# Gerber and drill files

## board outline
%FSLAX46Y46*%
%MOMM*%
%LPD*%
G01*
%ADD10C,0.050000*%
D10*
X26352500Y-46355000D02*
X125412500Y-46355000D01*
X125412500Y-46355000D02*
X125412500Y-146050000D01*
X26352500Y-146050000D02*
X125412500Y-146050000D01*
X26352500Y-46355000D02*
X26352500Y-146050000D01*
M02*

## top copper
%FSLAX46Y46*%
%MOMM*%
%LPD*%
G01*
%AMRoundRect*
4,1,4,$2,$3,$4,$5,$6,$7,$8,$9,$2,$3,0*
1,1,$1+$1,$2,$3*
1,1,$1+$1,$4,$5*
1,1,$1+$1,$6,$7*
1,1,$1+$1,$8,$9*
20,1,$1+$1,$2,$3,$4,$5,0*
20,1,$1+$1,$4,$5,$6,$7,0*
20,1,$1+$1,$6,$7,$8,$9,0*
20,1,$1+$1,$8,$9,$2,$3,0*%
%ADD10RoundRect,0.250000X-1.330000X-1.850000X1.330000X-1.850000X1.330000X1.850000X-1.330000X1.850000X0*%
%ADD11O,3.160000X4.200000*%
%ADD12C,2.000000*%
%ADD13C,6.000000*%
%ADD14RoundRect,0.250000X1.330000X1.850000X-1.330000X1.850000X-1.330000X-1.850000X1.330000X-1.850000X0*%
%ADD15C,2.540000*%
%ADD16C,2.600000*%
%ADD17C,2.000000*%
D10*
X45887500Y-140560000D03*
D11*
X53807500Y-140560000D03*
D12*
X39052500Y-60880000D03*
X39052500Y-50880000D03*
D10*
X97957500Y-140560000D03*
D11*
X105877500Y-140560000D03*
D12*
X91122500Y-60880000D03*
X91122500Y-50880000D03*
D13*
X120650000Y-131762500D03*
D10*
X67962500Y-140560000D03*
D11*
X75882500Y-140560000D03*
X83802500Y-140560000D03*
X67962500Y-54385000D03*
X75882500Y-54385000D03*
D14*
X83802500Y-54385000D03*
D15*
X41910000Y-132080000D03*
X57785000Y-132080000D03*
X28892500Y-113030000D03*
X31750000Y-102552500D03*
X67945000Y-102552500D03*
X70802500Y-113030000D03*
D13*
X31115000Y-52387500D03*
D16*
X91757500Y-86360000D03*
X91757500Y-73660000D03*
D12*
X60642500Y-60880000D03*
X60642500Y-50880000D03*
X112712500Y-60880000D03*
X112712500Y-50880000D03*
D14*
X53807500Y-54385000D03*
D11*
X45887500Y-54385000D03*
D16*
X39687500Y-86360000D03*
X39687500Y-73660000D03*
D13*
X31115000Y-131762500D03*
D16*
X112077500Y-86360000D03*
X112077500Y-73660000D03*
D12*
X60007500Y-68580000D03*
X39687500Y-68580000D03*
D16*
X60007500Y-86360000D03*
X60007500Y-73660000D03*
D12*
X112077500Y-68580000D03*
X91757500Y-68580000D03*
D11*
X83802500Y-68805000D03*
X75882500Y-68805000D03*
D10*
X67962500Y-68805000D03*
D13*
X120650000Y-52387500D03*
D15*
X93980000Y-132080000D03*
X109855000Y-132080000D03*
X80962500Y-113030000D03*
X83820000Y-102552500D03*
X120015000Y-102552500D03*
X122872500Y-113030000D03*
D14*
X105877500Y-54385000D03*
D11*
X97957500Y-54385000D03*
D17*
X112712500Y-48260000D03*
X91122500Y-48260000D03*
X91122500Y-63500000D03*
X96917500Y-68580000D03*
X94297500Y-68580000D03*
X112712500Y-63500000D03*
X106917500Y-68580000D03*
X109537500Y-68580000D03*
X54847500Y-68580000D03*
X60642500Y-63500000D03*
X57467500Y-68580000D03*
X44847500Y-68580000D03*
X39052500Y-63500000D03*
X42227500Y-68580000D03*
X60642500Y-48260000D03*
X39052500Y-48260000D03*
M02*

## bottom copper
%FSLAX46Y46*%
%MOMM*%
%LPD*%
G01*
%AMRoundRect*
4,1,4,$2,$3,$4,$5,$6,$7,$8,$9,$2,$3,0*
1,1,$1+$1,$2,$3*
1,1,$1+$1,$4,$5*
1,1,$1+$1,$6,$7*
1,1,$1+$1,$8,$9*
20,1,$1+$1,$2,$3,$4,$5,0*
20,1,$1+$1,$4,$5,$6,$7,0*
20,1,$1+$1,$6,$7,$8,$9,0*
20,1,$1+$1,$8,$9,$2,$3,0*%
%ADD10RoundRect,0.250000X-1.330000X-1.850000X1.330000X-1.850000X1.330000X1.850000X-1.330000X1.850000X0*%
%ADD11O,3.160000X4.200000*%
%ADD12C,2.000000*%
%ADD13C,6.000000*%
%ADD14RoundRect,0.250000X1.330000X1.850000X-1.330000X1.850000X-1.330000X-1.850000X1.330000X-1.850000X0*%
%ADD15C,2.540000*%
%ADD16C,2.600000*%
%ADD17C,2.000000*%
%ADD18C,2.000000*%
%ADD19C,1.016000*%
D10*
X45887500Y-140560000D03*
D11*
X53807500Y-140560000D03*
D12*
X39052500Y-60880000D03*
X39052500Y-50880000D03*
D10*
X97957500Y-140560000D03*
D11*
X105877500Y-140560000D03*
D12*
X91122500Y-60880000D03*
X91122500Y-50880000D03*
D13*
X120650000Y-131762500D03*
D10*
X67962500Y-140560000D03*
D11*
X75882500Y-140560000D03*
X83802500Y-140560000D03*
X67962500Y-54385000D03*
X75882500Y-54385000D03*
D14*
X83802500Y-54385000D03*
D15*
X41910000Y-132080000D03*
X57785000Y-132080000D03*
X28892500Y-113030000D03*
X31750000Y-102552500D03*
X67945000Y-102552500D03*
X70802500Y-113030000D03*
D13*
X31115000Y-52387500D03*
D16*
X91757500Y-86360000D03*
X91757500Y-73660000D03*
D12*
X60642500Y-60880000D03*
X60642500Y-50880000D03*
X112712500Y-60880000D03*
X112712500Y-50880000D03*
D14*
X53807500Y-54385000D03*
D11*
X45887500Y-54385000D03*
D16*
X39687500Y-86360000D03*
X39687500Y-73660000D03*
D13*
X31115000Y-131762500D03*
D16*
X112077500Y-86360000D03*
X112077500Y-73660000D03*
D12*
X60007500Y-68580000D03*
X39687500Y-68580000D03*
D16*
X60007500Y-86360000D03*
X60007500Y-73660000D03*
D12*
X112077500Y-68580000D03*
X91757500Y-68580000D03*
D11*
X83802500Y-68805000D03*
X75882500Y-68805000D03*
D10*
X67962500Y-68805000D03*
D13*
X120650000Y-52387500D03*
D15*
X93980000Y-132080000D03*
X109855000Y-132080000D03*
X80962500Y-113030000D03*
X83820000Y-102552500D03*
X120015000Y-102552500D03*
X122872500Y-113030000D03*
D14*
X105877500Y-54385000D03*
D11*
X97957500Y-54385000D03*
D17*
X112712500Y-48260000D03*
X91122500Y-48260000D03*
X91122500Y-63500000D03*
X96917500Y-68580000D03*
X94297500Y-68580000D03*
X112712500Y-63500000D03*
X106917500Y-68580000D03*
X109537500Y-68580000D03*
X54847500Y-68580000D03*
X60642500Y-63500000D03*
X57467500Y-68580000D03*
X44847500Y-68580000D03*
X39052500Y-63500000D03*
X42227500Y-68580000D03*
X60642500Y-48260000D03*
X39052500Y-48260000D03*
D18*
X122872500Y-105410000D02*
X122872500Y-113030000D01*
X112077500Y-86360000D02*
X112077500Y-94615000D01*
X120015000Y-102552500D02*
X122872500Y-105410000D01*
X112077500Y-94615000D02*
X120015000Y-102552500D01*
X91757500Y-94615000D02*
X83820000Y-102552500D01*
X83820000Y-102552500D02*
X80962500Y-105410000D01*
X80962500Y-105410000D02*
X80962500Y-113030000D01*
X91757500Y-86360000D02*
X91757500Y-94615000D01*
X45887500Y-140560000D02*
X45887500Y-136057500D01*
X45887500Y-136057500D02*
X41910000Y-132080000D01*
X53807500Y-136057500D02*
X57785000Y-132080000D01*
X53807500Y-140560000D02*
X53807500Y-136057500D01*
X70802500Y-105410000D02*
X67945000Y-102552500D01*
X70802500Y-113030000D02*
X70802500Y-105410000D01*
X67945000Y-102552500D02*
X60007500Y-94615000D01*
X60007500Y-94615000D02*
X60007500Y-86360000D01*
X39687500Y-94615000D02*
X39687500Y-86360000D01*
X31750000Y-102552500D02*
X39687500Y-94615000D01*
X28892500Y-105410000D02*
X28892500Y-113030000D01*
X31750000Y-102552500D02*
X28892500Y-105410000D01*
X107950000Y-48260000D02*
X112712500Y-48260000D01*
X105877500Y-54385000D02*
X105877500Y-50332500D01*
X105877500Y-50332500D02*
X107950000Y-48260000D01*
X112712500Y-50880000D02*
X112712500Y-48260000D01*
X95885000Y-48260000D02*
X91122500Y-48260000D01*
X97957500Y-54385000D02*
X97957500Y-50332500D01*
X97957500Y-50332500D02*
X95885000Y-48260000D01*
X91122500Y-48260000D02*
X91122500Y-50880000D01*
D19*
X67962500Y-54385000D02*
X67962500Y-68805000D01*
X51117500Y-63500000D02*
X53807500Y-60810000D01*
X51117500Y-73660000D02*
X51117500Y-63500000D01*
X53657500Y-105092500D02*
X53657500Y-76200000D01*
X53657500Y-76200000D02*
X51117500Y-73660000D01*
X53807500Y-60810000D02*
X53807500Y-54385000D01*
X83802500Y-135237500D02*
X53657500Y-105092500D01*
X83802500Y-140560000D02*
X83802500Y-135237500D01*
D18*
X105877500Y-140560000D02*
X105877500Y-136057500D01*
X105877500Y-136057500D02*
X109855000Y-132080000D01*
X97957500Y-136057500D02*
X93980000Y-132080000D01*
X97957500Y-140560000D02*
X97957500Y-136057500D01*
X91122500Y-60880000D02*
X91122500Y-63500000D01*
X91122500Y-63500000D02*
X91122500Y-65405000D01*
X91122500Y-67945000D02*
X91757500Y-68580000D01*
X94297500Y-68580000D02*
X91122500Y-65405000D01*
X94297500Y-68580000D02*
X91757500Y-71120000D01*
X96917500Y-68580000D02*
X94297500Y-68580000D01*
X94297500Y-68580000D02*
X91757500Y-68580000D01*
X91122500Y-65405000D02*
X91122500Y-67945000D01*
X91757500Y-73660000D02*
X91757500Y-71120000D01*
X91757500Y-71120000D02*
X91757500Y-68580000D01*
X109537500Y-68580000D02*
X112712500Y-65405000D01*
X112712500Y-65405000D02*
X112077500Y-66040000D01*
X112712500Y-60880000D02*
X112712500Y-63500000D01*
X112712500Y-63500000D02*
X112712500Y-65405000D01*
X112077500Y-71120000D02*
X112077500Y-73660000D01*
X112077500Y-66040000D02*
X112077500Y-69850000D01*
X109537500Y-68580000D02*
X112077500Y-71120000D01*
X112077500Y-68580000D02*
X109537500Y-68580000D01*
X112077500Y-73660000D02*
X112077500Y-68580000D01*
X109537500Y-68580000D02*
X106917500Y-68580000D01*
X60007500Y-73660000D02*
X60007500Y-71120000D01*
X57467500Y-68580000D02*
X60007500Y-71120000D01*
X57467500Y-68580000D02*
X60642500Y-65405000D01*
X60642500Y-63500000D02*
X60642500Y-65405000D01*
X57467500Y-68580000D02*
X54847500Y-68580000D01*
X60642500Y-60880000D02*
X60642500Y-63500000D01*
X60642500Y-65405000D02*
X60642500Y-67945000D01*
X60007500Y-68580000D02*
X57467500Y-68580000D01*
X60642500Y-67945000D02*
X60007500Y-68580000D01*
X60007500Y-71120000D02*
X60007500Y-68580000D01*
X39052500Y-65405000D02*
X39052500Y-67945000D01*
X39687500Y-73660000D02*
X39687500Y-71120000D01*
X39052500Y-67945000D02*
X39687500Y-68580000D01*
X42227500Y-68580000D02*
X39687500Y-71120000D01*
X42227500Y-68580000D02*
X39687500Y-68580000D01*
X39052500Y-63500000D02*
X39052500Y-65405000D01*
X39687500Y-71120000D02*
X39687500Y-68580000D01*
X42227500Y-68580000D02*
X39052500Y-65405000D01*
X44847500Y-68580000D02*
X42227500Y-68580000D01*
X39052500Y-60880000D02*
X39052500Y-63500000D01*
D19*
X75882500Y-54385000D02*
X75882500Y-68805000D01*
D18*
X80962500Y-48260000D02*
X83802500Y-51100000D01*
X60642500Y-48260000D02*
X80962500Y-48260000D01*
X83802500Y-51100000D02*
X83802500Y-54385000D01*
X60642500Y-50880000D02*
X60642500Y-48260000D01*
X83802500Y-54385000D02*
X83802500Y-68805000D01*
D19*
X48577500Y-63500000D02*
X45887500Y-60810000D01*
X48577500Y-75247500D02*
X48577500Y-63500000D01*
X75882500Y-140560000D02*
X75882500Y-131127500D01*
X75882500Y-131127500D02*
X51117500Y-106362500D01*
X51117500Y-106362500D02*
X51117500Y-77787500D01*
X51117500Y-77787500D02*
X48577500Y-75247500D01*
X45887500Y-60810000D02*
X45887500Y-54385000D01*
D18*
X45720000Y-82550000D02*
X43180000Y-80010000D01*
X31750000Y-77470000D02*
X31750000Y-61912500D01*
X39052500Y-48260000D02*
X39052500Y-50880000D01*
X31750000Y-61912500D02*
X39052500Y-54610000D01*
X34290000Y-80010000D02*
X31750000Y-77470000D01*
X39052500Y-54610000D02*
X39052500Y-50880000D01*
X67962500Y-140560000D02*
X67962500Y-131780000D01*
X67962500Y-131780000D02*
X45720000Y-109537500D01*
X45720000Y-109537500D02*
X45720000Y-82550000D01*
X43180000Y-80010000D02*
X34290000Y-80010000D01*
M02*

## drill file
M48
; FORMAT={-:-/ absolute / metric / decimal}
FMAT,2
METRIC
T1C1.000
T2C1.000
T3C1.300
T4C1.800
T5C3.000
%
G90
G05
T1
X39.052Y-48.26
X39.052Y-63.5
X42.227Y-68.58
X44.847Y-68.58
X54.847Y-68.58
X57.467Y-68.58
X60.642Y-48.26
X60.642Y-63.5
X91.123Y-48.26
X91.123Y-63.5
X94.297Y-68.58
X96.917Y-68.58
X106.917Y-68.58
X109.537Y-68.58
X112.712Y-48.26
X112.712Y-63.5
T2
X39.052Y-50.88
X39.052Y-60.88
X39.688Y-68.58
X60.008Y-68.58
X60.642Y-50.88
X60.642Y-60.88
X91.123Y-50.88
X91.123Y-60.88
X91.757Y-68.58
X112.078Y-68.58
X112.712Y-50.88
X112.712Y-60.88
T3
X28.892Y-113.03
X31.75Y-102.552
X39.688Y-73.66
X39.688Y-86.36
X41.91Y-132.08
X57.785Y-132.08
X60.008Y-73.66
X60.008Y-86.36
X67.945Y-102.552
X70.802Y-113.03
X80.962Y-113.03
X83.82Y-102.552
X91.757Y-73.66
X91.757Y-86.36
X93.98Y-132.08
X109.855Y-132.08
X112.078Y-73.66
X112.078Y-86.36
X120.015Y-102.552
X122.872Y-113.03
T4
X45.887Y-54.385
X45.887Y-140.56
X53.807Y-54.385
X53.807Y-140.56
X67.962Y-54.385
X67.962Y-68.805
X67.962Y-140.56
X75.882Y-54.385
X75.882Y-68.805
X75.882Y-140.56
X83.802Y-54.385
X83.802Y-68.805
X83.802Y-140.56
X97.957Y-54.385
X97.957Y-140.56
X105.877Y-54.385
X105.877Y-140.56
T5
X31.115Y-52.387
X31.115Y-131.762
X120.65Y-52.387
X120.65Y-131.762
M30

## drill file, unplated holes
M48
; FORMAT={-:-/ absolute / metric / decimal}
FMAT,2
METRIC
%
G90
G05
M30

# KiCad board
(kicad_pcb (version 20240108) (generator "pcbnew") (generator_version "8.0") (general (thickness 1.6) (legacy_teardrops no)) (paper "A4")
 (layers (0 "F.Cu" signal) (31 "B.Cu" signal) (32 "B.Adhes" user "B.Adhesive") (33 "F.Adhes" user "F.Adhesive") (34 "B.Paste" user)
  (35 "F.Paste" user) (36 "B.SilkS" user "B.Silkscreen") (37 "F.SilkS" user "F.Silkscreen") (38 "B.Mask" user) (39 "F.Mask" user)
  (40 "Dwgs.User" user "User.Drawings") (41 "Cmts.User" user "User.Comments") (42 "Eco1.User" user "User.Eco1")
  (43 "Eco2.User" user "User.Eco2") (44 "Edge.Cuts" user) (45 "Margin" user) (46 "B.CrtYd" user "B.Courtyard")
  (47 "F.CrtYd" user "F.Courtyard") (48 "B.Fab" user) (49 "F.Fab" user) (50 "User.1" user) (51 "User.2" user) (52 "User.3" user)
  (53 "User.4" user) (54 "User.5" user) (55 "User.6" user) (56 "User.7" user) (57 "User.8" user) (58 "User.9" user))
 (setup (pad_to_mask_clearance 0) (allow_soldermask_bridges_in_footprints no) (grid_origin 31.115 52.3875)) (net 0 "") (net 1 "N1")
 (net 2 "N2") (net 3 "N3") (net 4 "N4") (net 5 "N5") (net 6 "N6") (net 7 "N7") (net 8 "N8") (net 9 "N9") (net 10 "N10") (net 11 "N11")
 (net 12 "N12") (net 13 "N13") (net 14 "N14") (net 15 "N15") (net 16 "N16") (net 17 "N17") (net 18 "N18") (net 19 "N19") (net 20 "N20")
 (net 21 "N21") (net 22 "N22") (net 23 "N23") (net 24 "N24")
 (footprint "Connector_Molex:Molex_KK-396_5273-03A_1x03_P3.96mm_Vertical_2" (layer "F.Cu") (at 45.8875 140.56)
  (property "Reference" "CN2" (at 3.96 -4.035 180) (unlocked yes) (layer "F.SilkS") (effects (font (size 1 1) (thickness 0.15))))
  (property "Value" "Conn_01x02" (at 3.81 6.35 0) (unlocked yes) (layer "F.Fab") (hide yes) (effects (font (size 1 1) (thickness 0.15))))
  (pad "1" thru_hole roundrect (at 0 0) (size 3.16 4.2) (drill 1.8) (layers "*.Cu" "*.Mask") (remove_unused_layers no)
   (roundrect_rratio 0.079114) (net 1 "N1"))
  (pad "2" thru_hole oval (at 7.92 0) (size 3.16 4.2) (drill 1.8) (layers "*.Cu" "*.Mask") (remove_unused_layers no) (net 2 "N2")))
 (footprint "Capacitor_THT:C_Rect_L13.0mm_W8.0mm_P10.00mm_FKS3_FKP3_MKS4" (layer "F.Cu") (at 39.0525 60.88 90)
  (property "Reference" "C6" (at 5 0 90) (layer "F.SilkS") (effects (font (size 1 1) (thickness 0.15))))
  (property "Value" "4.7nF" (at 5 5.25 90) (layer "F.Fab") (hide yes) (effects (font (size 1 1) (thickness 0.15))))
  (pad "1" thru_hole circle (at 0 0 90) (size 2 2) (drill 1) (layers "*.Cu" "*.Mask") (remove_unused_layers no) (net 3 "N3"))
  (pad "2" thru_hole circle (at 10 0 90) (size 2 2) (drill 1) (layers "*.Cu" "*.Mask") (remove_unused_layers no) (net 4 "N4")))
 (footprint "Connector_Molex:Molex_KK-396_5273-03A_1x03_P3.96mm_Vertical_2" (layer "F.Cu") (at 97.9575 140.56)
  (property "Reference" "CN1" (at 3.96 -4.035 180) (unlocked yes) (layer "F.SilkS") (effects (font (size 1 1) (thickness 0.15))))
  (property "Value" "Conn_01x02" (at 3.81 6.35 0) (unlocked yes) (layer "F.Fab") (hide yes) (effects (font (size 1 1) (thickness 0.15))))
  (pad "1" thru_hole roundrect (at 0 0) (size 3.16 4.2) (drill 1.8) (layers "*.Cu" "*.Mask") (remove_unused_layers no)
   (roundrect_rratio 0.079114) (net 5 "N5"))
  (pad "2" thru_hole oval (at 7.92 0) (size 3.16 4.2) (drill 1.8) (layers "*.Cu" "*.Mask") (remove_unused_layers no) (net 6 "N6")))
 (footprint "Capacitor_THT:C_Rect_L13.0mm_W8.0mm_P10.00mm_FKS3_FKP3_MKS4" (layer "F.Cu") (at 91.1225 60.88 90)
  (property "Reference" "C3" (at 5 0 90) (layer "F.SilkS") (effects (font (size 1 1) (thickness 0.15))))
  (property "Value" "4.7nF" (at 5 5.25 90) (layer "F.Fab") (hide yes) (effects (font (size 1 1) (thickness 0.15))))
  (pad "1" thru_hole circle (at 0 0 90) (size 2 2) (drill 1) (layers "*.Cu" "*.Mask") (remove_unused_layers no) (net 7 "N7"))
  (pad "2" thru_hole circle (at 10 0 90) (size 2 2) (drill 1) (layers "*.Cu" "*.Mask") (remove_unused_layers no) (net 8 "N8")))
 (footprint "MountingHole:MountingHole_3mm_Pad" (layer "F.Cu") (at 120.65 131.7625 -90)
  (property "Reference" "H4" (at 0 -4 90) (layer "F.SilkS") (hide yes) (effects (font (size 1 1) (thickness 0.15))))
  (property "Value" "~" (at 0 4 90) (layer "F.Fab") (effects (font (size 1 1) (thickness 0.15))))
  (pad "1" thru_hole circle (at 0 0 270) (size 6 6) (drill 3) (layers "*.Cu" "*.Mask") (remove_unused_layers no) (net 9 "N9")))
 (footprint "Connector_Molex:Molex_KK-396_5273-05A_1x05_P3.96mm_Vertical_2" (layer "F.Cu") (at 67.9625 140.56)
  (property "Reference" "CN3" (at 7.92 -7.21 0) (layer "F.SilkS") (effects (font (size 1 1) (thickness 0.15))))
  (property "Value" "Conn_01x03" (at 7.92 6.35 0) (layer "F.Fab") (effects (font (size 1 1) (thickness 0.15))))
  (pad "1" thru_hole roundrect (at 0 0) (size 3.16 4.2) (drill 1.8) (layers "*.Cu" "*.Mask") (remove_unused_layers no)
   (roundrect_rratio 0.079114) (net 4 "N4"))
  (pad "2" thru_hole oval (at 7.92 0) (size 3.16 4.2) (drill 1.8) (layers "*.Cu" "*.Mask") (remove_unused_layers no) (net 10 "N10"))
  (pad "3" thru_hole oval (at 15.84 0) (size 3.16 4.2) (drill 1.8) (layers "*.Cu" "*.Mask") (remove_unused_layers no) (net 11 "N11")))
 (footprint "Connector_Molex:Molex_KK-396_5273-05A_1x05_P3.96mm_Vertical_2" (layer "F.Cu") (at 83.8025 54.385 180)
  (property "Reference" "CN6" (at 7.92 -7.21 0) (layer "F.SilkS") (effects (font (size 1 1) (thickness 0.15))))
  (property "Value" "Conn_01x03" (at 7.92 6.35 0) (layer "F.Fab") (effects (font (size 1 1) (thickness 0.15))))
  (pad "1" thru_hole roundrect (at 0 0 180) (size 3.16 4.2) (drill 1.8) (layers "*.Cu" "*.Mask") (remove_unused_layers no)
   (roundrect_rratio 0.079114) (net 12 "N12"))
  (pad "2" thru_hole oval (at 7.92 0 180) (size 3.16 4.2) (drill 1.8) (layers "*.Cu" "*.Mask") (remove_unused_layers no) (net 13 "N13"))
  (pad "3" thru_hole oval (at 15.84 0 180) (size 3.16 4.2) (drill 1.8) (layers "*.Cu" "*.Mask") (remove_unused_layers no) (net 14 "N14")))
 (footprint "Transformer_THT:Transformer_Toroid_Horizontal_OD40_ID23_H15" (layer "F.Cu") (at 49.8475 113.03)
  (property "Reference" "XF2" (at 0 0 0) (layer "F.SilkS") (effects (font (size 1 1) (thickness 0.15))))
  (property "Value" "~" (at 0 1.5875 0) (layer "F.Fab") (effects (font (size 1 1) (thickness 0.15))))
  (pad "1" thru_hole circle (at -7.9375 19.05) (size 2.54 2.54) (drill 1.3) (layers "*.Cu" "*.Mask") (remove_unused_layers no) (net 1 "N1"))
  (pad "2" thru_hole circle (at 7.9375 19.05) (size 2.54 2.54) (drill 1.3) (layers "*.Cu" "*.Mask") (remove_unused_layers no) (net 2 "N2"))
  (pad "3" thru_hole circle (at -20.955 0) (size 2.54 2.54) (drill 1.3) (layers "*.Cu" "*.Mask") (remove_unused_layers no) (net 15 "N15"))
  (pad "3" thru_hole circle (at -18.0975 -10.4775) (size 2.54 2.54) (drill 1.3) (layers "*.Cu" "*.Mask") (remove_unused_layers no)
   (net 15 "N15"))
  (pad "4" thru_hole circle (at 18.0975 -10.4775) (size 2.54 2.54) (drill 1.3) (layers "*.Cu" "*.Mask") (remove_unused_layers no)
   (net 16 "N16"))
  (pad "4" thru_hole circle (at 20.955 0) (size 2.54 2.54) (drill 1.3) (layers "*.Cu" "*.Mask") (remove_unused_layers no) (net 16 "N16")))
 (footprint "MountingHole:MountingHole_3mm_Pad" (layer "F.Cu") (at 31.115 52.3875 -90)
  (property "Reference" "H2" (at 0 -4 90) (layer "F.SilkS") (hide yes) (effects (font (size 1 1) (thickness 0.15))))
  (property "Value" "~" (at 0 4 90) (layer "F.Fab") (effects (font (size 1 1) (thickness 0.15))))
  (pad "1" thru_hole circle (at 0 0 270) (size 6 6) (drill 3) (layers "*.Cu" "*.Mask") (remove_unused_layers no) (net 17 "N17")))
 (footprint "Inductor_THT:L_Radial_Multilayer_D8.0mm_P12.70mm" (layer "F.Cu") (at 91.7575 81.915 90)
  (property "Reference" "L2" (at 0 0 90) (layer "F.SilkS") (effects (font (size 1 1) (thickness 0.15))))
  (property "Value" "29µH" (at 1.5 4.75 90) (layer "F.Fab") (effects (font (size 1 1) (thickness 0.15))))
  (pad "1" thru_hole circle (at -4.445 0 90) (size 2.6 2.6) (drill 1.3) (layers "*.Cu" "*.Mask") (remove_unused_layers no) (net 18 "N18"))
  (pad "2" thru_hole circle (at 8.255 0 90) (size 2.6 2.6) (drill 1.3) (layers "*.Cu" "*.Mask") (remove_unused_layers no) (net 7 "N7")))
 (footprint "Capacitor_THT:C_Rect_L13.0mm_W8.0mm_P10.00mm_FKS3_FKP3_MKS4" (layer "F.Cu") (at 60.6425 60.88 90)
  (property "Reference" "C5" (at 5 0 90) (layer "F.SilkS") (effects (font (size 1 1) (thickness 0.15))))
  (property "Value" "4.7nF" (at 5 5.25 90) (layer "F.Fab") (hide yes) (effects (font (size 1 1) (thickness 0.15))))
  (pad "1" thru_hole circle (at 0 0 90) (size 2 2) (drill 1) (layers "*.Cu" "*.Mask") (remove_unused_layers no) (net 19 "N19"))
  (pad "2" thru_hole circle (at 10 0 90) (size 2 2) (drill 1) (layers "*.Cu" "*.Mask") (remove_unused_layers no) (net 12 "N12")))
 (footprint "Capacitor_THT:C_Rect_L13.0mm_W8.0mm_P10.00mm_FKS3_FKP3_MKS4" (layer "F.Cu") (at 112.7125 60.88 90)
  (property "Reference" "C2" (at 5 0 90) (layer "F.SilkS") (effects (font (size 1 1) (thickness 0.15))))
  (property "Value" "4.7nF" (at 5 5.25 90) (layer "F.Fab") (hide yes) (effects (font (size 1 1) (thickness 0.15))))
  (pad "1" thru_hole circle (at 0 0 90) (size 2 2) (drill 1) (layers "*.Cu" "*.Mask") (remove_unused_layers no) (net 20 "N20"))
  (pad "2" thru_hole circle (at 10 0 90) (size 2 2) (drill 1) (layers "*.Cu" "*.Mask") (remove_unused_layers no) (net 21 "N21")))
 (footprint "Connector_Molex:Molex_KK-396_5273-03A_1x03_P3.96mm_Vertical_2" (layer "F.Cu") (at 53.8075 54.385 180)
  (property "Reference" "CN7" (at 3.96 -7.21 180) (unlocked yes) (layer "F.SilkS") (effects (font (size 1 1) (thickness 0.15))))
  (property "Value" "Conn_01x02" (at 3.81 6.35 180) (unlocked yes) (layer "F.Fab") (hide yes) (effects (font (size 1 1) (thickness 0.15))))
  (pad "1" thru_hole roundrect (at 0 0 180) (size 3.16 4.2) (drill 1.8) (layers "*.Cu" "*.Mask") (remove_unused_layers no)
   (roundrect_rratio 0.079114) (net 11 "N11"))
  (pad "2" thru_hole oval (at 7.92 0 180) (size 3.16 4.2) (drill 1.8) (layers "*.Cu" "*.Mask") (remove_unused_layers no) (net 10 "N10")))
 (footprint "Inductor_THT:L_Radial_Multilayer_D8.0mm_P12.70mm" (layer "F.Cu") (at 39.6875 81.915 90)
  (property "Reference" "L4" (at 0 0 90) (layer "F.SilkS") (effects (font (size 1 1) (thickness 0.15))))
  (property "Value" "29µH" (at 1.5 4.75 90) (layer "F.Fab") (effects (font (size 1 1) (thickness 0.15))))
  (pad "1" thru_hole circle (at -4.445 0 90) (size 2.6 2.6) (drill 1.3) (layers "*.Cu" "*.Mask") (remove_unused_layers no) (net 15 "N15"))
  (pad "2" thru_hole circle (at 8.255 0 90) (size 2.6 2.6) (drill 1.3) (layers "*.Cu" "*.Mask") (remove_unused_layers no) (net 3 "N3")))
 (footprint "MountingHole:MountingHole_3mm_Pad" (layer "F.Cu") (at 31.115 131.7625 -90)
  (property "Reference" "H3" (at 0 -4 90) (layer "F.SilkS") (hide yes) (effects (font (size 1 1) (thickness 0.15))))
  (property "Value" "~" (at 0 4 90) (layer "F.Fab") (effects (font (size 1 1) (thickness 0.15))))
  (pad "1" thru_hole circle (at 0 0 270) (size 6 6) (drill 3) (layers "*.Cu" "*.Mask") (remove_unused_layers no) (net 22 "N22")))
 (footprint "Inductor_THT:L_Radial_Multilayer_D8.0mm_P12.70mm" (layer "F.Cu") (at 112.0775 81.915 90)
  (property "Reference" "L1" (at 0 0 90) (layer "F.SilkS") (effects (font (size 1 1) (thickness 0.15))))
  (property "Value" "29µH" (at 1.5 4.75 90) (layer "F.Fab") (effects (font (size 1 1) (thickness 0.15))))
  (pad "1" thru_hole circle (at -4.445 0 90) (size 2.6 2.6) (drill 1.3) (layers "*.Cu" "*.Mask") (remove_unused_layers no) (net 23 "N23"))
  (pad "2" thru_hole circle (at 8.255 0 90) (size 2.6 2.6) (drill 1.3) (layers "*.Cu" "*.Mask") (remove_unused_layers no) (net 20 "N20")))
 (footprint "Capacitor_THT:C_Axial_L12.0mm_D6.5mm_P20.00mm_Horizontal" (layer "F.Cu") (at 59.8475 68.58 180)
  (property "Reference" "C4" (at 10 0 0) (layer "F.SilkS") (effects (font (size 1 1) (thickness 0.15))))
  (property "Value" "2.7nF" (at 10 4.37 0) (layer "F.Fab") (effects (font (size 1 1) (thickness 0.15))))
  (pad "1" thru_hole circle (at -0.16 0 180) (size 2 2) (drill 1) (layers "*.Cu" "*.Mask") (remove_unused_layers no) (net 19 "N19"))
  (pad "2" thru_hole circle (at 20.16 0 180) (size 2 2) (drill 1) (layers "*.Cu" "*.Mask") (remove_unused_layers no) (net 3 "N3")
   (thermal_bridge_angle 90)))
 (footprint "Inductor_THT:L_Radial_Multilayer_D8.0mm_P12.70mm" (layer "F.Cu") (at 60.0075 81.915 90)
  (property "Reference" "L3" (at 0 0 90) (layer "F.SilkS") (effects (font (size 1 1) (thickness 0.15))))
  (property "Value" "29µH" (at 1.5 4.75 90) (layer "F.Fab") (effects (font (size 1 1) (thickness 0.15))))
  (pad "1" thru_hole circle (at -4.445 0 90) (size 2.6 2.6) (drill 1.3) (layers "*.Cu" "*.Mask") (remove_unused_layers no) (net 16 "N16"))
  (pad "2" thru_hole circle (at 8.255 0 90) (size 2.6 2.6) (drill 1.3) (layers "*.Cu" "*.Mask") (remove_unused_layers no) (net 19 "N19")))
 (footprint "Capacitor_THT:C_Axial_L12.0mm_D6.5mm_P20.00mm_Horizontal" (layer "F.Cu") (at 111.9175 68.58 180)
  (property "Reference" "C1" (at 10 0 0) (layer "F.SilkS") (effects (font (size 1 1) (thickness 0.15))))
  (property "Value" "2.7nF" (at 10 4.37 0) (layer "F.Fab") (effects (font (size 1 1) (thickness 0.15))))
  (pad "1" thru_hole circle (at -0.16 0 180) (size 2 2) (drill 1) (layers "*.Cu" "*.Mask") (remove_unused_layers no) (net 20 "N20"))
  (pad "2" thru_hole circle (at 20.16 0 180) (size 2 2) (drill 1) (layers "*.Cu" "*.Mask") (remove_unused_layers no) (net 7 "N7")
   (thermal_bridge_angle 90)))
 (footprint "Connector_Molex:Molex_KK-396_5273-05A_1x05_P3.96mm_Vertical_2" (layer "F.Cu") (at 67.9625 68.805)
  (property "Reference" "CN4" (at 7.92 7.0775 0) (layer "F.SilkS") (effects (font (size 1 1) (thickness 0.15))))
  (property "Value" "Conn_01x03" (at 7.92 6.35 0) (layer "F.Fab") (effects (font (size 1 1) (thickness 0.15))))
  (pad "1" thru_hole roundrect (at 0 0) (size 3.16 4.2) (drill 1.8) (layers "*.Cu" "*.Mask") (remove_unused_layers no)
   (roundrect_rratio 0.079114) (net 14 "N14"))
  (pad "2" thru_hole oval (at 7.92 0) (size 3.16 4.2) (drill 1.8) (layers "*.Cu" "*.Mask") (remove_unused_layers no) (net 13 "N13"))
  (pad "3" thru_hole oval (at 15.84 0) (size 3.16 4.2) (drill 1.8) (layers "*.Cu" "*.Mask") (remove_unused_layers no) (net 12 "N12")))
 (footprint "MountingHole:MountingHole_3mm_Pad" (layer "F.Cu") (at 120.65 52.3875 -90)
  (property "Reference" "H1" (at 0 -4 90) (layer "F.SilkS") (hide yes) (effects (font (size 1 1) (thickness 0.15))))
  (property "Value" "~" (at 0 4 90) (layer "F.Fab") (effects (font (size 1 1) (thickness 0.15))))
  (pad "1" thru_hole circle (at 0 0 270) (size 6 6) (drill 3) (layers "*.Cu" "*.Mask") (remove_unused_layers no) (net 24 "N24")))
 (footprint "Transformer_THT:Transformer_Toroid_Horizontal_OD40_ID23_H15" (layer "F.Cu") (at 101.9175 113.03)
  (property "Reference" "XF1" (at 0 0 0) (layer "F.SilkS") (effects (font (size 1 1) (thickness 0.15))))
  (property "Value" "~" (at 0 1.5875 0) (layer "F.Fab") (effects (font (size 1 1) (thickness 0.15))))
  (pad "1" thru_hole circle (at -7.9375 19.05) (size 2.54 2.54) (drill 1.3) (layers "*.Cu" "*.Mask") (remove_unused_layers no) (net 5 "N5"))
  (pad "2" thru_hole circle (at 7.9375 19.05) (size 2.54 2.54) (drill 1.3) (layers "*.Cu" "*.Mask") (remove_unused_layers no) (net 6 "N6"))
  (pad "3" thru_hole circle (at -20.955 0) (size 2.54 2.54) (drill 1.3) (layers "*.Cu" "*.Mask") (remove_unused_layers no) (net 18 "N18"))
  (pad "3" thru_hole circle (at -18.0975 -10.4775) (size 2.54 2.54) (drill 1.3) (layers "*.Cu" "*.Mask") (remove_unused_layers no)
   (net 18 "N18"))
  (pad "4" thru_hole circle (at 18.0975 -10.4775) (size 2.54 2.54) (drill 1.3) (layers "*.Cu" "*.Mask") (remove_unused_layers no)
   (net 23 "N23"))
  (pad "4" thru_hole circle (at 20.955 0) (size 2.54 2.54) (drill 1.3) (layers "*.Cu" "*.Mask") (remove_unused_layers no) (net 23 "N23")))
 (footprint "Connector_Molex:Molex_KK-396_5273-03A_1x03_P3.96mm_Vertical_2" (layer "F.Cu") (at 105.8775 54.385 180)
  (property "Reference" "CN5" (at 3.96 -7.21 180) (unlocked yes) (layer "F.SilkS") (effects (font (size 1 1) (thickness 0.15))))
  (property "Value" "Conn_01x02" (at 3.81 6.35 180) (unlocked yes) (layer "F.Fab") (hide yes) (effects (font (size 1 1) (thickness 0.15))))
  (pad "1" thru_hole roundrect (at 0 0 180) (size 3.16 4.2) (drill 1.8) (layers "*.Cu" "*.Mask") (remove_unused_layers no)
   (roundrect_rratio 0.079114) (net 21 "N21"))
  (pad "2" thru_hole oval (at 7.92 0 180) (size 3.16 4.2) (drill 1.8) (layers "*.Cu" "*.Mask") (remove_unused_layers no) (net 8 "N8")))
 (gr_line (start 26.3525 46.355) (end 125.4125 46.355) (stroke (width 0.05) (type default)) (layer "Edge.Cuts"))
 (gr_line (start 125.4125 46.355) (end 125.4125 146.05) (stroke (width 0.05) (type default)) (layer "Edge.Cuts"))
 (gr_line (start 26.3525 146.05) (end 125.4125 146.05) (stroke (width 0.05) (type default)) (layer "Edge.Cuts"))
 (gr_line (start 26.3525 46.355) (end 26.3525 146.05) (stroke (width 0.05) (type default)) (layer "Edge.Cuts"))
 (segment (start 122.8725 105.41) (end 122.8725 113.03) (width 2) (layer "B.Cu") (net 23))
 (segment (start 112.0775 86.36) (end 112.0775 94.615) (width 2) (layer "B.Cu") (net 23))
 (segment (start 120.015 102.5525) (end 122.8725 105.41) (width 2) (layer "B.Cu") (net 23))
 (segment (start 112.0775 94.615) (end 120.015 102.5525) (width 2) (layer "B.Cu") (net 23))
 (segment (start 91.7575 94.615) (end 83.82 102.5525) (width 2) (layer "B.Cu") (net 18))
 (segment (start 83.82 102.5525) (end 80.9625 105.41) (width 2) (layer "B.Cu") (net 18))
 (segment (start 80.9625 105.41) (end 80.9625 113.03) (width 2) (layer "B.Cu") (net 18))
 (segment (start 91.7575 86.36) (end 91.7575 94.615) (width 2) (layer "B.Cu") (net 18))
 (segment (start 45.8875 140.56) (end 45.8875 136.0575) (width 2) (layer "B.Cu") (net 1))
 (segment (start 45.8875 136.0575) (end 41.91 132.08) (width 2) (layer "B.Cu") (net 1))
 (segment (start 53.8075 136.0575) (end 57.785 132.08) (width 2) (layer "B.Cu") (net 2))
 (segment (start 53.8075 140.56) (end 53.8075 136.0575) (width 2) (layer "B.Cu") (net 2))
 (segment (start 70.8025 105.41) (end 67.945 102.5525) (width 2) (layer "B.Cu") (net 16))
 (segment (start 70.8025 113.03) (end 70.8025 105.41) (width 2) (layer "B.Cu") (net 16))
 (segment (start 67.945 102.5525) (end 60.0075 94.615) (width 2) (layer "B.Cu") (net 16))
 (segment (start 60.0075 94.615) (end 60.0075 86.36) (width 2) (layer "B.Cu") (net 16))
 (segment (start 39.6875 94.615) (end 39.6875 86.36) (width 2) (layer "B.Cu") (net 15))
 (segment (start 31.75 102.5525) (end 39.6875 94.615) (width 2) (layer "B.Cu") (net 15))
 (segment (start 28.8925 105.41) (end 28.8925 113.03) (width 2) (layer "B.Cu") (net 15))
 (segment (start 31.75 102.5525) (end 28.8925 105.41) (width 2) (layer "B.Cu") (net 15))
 (via (at 112.7125 48.26) (size 2) (drill 1) (layers "F.Cu" "B.Cu") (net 21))
 (segment (start 107.95 48.26) (end 112.7125 48.26) (width 2) (layer "B.Cu") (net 21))
 (segment (start 105.8775 54.385) (end 105.8775 50.3325) (width 2) (layer "B.Cu") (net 21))
 (segment (start 105.8775 50.3325) (end 107.95 48.26) (width 2) (layer "B.Cu") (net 21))
 (segment (start 112.7125 50.88) (end 112.7125 48.26) (width 2) (layer "B.Cu") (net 21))
 (via (at 91.1225 48.26) (size 2) (drill 1) (layers "F.Cu" "B.Cu") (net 8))
 (segment (start 95.885 48.26) (end 91.1225 48.26) (width 2) (layer "B.Cu") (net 8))
 (segment (start 97.9575 54.385) (end 97.9575 50.3325) (width 2) (layer "B.Cu") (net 8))
 (segment (start 97.9575 50.3325) (end 95.885 48.26) (width 2) (layer "B.Cu") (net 8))
 (segment (start 91.1225 48.26) (end 91.1225 50.88) (width 2) (layer "B.Cu") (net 8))
 (segment (start 67.9625 54.385) (end 67.9625 68.805) (width 1.016) (layer "B.Cu") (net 14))
 (segment (start 51.1175 63.5) (end 53.8075 60.81) (width 1.016) (layer "B.Cu") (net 11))
 (segment (start 51.1175 73.66) (end 51.1175 63.5) (width 1.016) (layer "B.Cu") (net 11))
 (segment (start 53.6575 105.0925) (end 53.6575 76.2) (width 1.016) (layer "B.Cu") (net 11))
 (segment (start 53.6575 76.2) (end 51.1175 73.66) (width 1.016) (layer "B.Cu") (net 11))
 (segment (start 53.8075 60.81) (end 53.8075 54.385) (width 1.016) (layer "B.Cu") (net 11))
 (segment (start 83.8025 135.2375) (end 53.6575 105.0925) (width 1.016) (layer "B.Cu") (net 11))
 (segment (start 83.8025 140.56) (end 83.8025 135.2375) (width 1.016) (layer "B.Cu") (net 11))
 (segment (start 105.8775 140.56) (end 105.8775 136.0575) (width 2) (layer "B.Cu") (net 6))
 (segment (start 105.8775 136.0575) (end 109.855 132.08) (width 2) (layer "B.Cu") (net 6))
 (segment (start 97.9575 136.0575) (end 93.98 132.08) (width 2) (layer "B.Cu") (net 5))
 (segment (start 97.9575 140.56) (end 97.9575 136.0575) (width 2) (layer "B.Cu") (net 5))
 (via (at 91.1225 63.5) (size 2) (drill 1) (layers "F.Cu" "B.Cu") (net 7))
 (via (at 96.9175 68.58) (size 2) (drill 1) (layers "F.Cu" "B.Cu") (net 7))
 (via (at 94.2975 68.58) (size 2) (drill 1) (layers "F.Cu" "B.Cu") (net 7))
 (segment (start 91.1225 60.88) (end 91.1225 63.5) (width 2) (layer "B.Cu") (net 7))
 (segment (start 91.1225 63.5) (end 91.1225 65.405) (width 2) (layer "B.Cu") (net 7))
 (segment (start 91.1225 67.945) (end 91.7575 68.58) (width 2) (layer "B.Cu") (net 7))
 (segment (start 94.2975 68.58) (end 91.1225 65.405) (width 2) (layer "B.Cu") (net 7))
 (segment (start 94.2975 68.58) (end 91.7575 71.12) (width 2) (layer "B.Cu") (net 7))
 (segment (start 96.9175 68.58) (end 94.2975 68.58) (width 2) (layer "B.Cu") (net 7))
 (segment (start 94.2975 68.58) (end 91.7575 68.58) (width 2) (layer "B.Cu") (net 7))
 (segment (start 91.1225 65.405) (end 91.1225 67.945) (width 2) (layer "B.Cu") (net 7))
 (segment (start 91.7575 73.66) (end 91.7575 71.12) (width 2) (layer "B.Cu") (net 7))
 (segment (start 91.7575 71.12) (end 91.7575 68.58) (width 2) (layer "B.Cu") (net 7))
 (via (at 112.7125 63.5) (size 2) (drill 1) (layers "F.Cu" "B.Cu") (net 20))
 (via (at 106.9175 68.58) (size 2) (drill 1) (layers "F.Cu" "B.Cu") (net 20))
 (via (at 109.5375 68.58) (size 2) (drill 1) (layers "F.Cu" "B.Cu") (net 20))
 (segment (start 109.5375 68.58) (end 112.7125 65.405) (width 2) (layer "B.Cu") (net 20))
 (segment (start 112.7125 65.405) (end 112.0775 66.04) (width 2) (layer "B.Cu") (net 20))
 (segment (start 112.7125 60.88) (end 112.7125 63.5) (width 2) (layer "B.Cu") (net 20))
 (segment (start 112.7125 63.5) (end 112.7125 65.405) (width 2) (layer "B.Cu") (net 20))
 (segment (start 112.0775 71.12) (end 112.0775 73.66) (width 2) (layer "B.Cu") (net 20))
 (segment (start 112.0775 66.04) (end 112.0775 69.85) (width 2) (layer "B.Cu") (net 20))
 (segment (start 109.5375 68.58) (end 112.0775 71.12) (width 2) (layer "B.Cu") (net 20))
 (segment (start 112.0775 68.58) (end 109.5375 68.58) (width 2) (layer "B.Cu") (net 20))
 (segment (start 112.0775 73.66) (end 112.0775 68.58) (width 2) (layer "B.Cu") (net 20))
 (segment (start 109.5375 68.58) (end 106.9175 68.58) (width 2) (layer "B.Cu") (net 20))
 (via (at 54.8475 68.58) (size 2) (drill 1) (layers "F.Cu" "B.Cu") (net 19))
 (via (at 60.6425 63.5) (size 2) (drill 1) (layers "F.Cu" "B.Cu") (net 19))
 (via (at 57.4675 68.58) (size 2) (drill 1) (layers "F.Cu" "B.Cu") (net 19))
 (segment (start 60.0075 73.66) (end 60.0075 71.12) (width 2) (layer "B.Cu") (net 19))
 (segment (start 57.4675 68.58) (end 60.0075 71.12) (width 2) (layer "B.Cu") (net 19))
 (segment (start 57.4675 68.58) (end 60.6425 65.405) (width 2) (layer "B.Cu") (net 19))
 (segment (start 60.6425 63.5) (end 60.6425 65.405) (width 2) (layer "B.Cu") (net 19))
 (segment (start 57.4675 68.58) (end 54.8475 68.58) (width 2) (layer "B.Cu") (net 19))
 (segment (start 60.6425 60.88) (end 60.6425 63.5) (width 2) (layer "B.Cu") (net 19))
 (segment (start 60.6425 65.405) (end 60.6425 67.945) (width 2) (layer "B.Cu") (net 19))
 (segment (start 60.0075 68.58) (end 57.4675 68.58) (width 2) (layer "B.Cu") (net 19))
 (segment (start 60.6425 67.945) (end 60.0075 68.58) (width 2) (layer "B.Cu") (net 19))
 (segment (start 60.0075 71.12) (end 60.0075 68.58) (width 2) (layer "B.Cu") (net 19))
 (via (at 44.8475 68.58) (size 2) (drill 1) (layers "F.Cu" "B.Cu") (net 3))
 (via (at 39.0525 63.5) (size 2) (drill 1) (layers "F.Cu" "B.Cu") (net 3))
 (via (at 42.2275 68.58) (size 2) (drill 1) (layers "F.Cu" "B.Cu") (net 3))
 (segment (start 39.0525 65.405) (end 39.0525 67.945) (width 2) (layer "B.Cu") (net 3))
 (segment (start 39.6875 73.66) (end 39.6875 71.12) (width 2) (layer "B.Cu") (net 3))
 (segment (start 39.0525 67.945) (end 39.6875 68.58) (width 2) (layer "B.Cu") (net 3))
 (segment (start 42.2275 68.58) (end 39.6875 71.12) (width 2) (layer "B.Cu") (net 3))
 (segment (start 42.2275 68.58) (end 39.6875 68.58) (width 2) (layer "B.Cu") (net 3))
 (segment (start 39.0525 63.5) (end 39.0525 65.405) (width 2) (layer "B.Cu") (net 3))
 (segment (start 39.6875 71.12) (end 39.6875 68.58) (width 2) (layer "B.Cu") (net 3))
 (segment (start 42.2275 68.58) (end 39.0525 65.405) (width 2) (layer "B.Cu") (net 3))
 (segment (start 44.8475 68.58) (end 42.2275 68.58) (width 2) (layer "B.Cu") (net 3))
 (segment (start 39.0525 60.88) (end 39.0525 63.5) (width 2) (layer "B.Cu") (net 3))
 (segment (start 75.8825 54.385) (end 75.8825 68.805) (width 1.016) (layer "B.Cu") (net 13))
 (via (at 60.6425 48.26) (size 2) (drill 1) (layers "F.Cu" "B.Cu") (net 12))
 (segment (start 80.9625 48.26) (end 83.8025 51.1) (width 2) (layer "B.Cu") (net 12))
 (segment (start 60.6425 48.26) (end 80.9625 48.26) (width 2) (layer "B.Cu") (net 12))
 (segment (start 83.8025 51.1) (end 83.8025 54.385) (width 2) (layer "B.Cu") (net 12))
 (segment (start 60.6425 50.88) (end 60.6425 48.26) (width 2) (layer "B.Cu") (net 12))
 (segment (start 83.8025 54.385) (end 83.8025 68.805) (width 2) (layer "B.Cu") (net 12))
 (segment (start 48.5775 63.5) (end 45.8875 60.81) (width 1.016) (layer "B.Cu") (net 10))
 (segment (start 48.5775 75.2475) (end 48.5775 63.5) (width 1.016) (layer "B.Cu") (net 10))
 (segment (start 75.8825 140.56) (end 75.8825 131.1275) (width 1.016) (layer "B.Cu") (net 10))
 (segment (start 75.8825 131.1275) (end 51.1175 106.3625) (width 1.016) (layer "B.Cu") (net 10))
 (segment (start 51.1175 106.3625) (end 51.1175 77.7875) (width 1.016) (layer "B.Cu") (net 10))
 (segment (start 51.1175 77.7875) (end 48.5775 75.2475) (width 1.016) (layer "B.Cu") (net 10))
 (segment (start 45.8875 60.81) (end 45.8875 54.385) (width 1.016) (layer "B.Cu") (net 10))
 (via (at 39.0525 48.26) (size 2) (drill 1) (layers "F.Cu" "B.Cu") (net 4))
 (segment (start 45.72 82.55) (end 43.18 80.01) (width 2) (layer "B.Cu") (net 4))
 (segment (start 31.75 77.47) (end 31.75 61.9125) (width 2) (layer "B.Cu") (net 4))
 (segment (start 39.0525 48.26) (end 39.0525 50.88) (width 2) (layer "B.Cu") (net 4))
 (segment (start 31.75 61.9125) (end 39.0525 54.61) (width 2) (layer "B.Cu") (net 4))
 (segment (start 34.29 80.01) (end 31.75 77.47) (width 2) (layer "B.Cu") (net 4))
 (segment (start 39.0525 54.61) (end 39.0525 50.88) (width 2) (layer "B.Cu") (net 4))
 (segment (start 67.9625 140.56) (end 67.9625 131.78) (width 2) (layer "B.Cu") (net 4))
 (segment (start 67.9625 131.78) (end 45.72 109.5375) (width 2) (layer "B.Cu") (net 4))
 (segment (start 45.72 109.5375) (end 45.72 82.55) (width 2) (layer "B.Cu") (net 4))
 (segment (start 43.18 80.01) (end 34.29 80.01) (width 2) (layer "B.Cu") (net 4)))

